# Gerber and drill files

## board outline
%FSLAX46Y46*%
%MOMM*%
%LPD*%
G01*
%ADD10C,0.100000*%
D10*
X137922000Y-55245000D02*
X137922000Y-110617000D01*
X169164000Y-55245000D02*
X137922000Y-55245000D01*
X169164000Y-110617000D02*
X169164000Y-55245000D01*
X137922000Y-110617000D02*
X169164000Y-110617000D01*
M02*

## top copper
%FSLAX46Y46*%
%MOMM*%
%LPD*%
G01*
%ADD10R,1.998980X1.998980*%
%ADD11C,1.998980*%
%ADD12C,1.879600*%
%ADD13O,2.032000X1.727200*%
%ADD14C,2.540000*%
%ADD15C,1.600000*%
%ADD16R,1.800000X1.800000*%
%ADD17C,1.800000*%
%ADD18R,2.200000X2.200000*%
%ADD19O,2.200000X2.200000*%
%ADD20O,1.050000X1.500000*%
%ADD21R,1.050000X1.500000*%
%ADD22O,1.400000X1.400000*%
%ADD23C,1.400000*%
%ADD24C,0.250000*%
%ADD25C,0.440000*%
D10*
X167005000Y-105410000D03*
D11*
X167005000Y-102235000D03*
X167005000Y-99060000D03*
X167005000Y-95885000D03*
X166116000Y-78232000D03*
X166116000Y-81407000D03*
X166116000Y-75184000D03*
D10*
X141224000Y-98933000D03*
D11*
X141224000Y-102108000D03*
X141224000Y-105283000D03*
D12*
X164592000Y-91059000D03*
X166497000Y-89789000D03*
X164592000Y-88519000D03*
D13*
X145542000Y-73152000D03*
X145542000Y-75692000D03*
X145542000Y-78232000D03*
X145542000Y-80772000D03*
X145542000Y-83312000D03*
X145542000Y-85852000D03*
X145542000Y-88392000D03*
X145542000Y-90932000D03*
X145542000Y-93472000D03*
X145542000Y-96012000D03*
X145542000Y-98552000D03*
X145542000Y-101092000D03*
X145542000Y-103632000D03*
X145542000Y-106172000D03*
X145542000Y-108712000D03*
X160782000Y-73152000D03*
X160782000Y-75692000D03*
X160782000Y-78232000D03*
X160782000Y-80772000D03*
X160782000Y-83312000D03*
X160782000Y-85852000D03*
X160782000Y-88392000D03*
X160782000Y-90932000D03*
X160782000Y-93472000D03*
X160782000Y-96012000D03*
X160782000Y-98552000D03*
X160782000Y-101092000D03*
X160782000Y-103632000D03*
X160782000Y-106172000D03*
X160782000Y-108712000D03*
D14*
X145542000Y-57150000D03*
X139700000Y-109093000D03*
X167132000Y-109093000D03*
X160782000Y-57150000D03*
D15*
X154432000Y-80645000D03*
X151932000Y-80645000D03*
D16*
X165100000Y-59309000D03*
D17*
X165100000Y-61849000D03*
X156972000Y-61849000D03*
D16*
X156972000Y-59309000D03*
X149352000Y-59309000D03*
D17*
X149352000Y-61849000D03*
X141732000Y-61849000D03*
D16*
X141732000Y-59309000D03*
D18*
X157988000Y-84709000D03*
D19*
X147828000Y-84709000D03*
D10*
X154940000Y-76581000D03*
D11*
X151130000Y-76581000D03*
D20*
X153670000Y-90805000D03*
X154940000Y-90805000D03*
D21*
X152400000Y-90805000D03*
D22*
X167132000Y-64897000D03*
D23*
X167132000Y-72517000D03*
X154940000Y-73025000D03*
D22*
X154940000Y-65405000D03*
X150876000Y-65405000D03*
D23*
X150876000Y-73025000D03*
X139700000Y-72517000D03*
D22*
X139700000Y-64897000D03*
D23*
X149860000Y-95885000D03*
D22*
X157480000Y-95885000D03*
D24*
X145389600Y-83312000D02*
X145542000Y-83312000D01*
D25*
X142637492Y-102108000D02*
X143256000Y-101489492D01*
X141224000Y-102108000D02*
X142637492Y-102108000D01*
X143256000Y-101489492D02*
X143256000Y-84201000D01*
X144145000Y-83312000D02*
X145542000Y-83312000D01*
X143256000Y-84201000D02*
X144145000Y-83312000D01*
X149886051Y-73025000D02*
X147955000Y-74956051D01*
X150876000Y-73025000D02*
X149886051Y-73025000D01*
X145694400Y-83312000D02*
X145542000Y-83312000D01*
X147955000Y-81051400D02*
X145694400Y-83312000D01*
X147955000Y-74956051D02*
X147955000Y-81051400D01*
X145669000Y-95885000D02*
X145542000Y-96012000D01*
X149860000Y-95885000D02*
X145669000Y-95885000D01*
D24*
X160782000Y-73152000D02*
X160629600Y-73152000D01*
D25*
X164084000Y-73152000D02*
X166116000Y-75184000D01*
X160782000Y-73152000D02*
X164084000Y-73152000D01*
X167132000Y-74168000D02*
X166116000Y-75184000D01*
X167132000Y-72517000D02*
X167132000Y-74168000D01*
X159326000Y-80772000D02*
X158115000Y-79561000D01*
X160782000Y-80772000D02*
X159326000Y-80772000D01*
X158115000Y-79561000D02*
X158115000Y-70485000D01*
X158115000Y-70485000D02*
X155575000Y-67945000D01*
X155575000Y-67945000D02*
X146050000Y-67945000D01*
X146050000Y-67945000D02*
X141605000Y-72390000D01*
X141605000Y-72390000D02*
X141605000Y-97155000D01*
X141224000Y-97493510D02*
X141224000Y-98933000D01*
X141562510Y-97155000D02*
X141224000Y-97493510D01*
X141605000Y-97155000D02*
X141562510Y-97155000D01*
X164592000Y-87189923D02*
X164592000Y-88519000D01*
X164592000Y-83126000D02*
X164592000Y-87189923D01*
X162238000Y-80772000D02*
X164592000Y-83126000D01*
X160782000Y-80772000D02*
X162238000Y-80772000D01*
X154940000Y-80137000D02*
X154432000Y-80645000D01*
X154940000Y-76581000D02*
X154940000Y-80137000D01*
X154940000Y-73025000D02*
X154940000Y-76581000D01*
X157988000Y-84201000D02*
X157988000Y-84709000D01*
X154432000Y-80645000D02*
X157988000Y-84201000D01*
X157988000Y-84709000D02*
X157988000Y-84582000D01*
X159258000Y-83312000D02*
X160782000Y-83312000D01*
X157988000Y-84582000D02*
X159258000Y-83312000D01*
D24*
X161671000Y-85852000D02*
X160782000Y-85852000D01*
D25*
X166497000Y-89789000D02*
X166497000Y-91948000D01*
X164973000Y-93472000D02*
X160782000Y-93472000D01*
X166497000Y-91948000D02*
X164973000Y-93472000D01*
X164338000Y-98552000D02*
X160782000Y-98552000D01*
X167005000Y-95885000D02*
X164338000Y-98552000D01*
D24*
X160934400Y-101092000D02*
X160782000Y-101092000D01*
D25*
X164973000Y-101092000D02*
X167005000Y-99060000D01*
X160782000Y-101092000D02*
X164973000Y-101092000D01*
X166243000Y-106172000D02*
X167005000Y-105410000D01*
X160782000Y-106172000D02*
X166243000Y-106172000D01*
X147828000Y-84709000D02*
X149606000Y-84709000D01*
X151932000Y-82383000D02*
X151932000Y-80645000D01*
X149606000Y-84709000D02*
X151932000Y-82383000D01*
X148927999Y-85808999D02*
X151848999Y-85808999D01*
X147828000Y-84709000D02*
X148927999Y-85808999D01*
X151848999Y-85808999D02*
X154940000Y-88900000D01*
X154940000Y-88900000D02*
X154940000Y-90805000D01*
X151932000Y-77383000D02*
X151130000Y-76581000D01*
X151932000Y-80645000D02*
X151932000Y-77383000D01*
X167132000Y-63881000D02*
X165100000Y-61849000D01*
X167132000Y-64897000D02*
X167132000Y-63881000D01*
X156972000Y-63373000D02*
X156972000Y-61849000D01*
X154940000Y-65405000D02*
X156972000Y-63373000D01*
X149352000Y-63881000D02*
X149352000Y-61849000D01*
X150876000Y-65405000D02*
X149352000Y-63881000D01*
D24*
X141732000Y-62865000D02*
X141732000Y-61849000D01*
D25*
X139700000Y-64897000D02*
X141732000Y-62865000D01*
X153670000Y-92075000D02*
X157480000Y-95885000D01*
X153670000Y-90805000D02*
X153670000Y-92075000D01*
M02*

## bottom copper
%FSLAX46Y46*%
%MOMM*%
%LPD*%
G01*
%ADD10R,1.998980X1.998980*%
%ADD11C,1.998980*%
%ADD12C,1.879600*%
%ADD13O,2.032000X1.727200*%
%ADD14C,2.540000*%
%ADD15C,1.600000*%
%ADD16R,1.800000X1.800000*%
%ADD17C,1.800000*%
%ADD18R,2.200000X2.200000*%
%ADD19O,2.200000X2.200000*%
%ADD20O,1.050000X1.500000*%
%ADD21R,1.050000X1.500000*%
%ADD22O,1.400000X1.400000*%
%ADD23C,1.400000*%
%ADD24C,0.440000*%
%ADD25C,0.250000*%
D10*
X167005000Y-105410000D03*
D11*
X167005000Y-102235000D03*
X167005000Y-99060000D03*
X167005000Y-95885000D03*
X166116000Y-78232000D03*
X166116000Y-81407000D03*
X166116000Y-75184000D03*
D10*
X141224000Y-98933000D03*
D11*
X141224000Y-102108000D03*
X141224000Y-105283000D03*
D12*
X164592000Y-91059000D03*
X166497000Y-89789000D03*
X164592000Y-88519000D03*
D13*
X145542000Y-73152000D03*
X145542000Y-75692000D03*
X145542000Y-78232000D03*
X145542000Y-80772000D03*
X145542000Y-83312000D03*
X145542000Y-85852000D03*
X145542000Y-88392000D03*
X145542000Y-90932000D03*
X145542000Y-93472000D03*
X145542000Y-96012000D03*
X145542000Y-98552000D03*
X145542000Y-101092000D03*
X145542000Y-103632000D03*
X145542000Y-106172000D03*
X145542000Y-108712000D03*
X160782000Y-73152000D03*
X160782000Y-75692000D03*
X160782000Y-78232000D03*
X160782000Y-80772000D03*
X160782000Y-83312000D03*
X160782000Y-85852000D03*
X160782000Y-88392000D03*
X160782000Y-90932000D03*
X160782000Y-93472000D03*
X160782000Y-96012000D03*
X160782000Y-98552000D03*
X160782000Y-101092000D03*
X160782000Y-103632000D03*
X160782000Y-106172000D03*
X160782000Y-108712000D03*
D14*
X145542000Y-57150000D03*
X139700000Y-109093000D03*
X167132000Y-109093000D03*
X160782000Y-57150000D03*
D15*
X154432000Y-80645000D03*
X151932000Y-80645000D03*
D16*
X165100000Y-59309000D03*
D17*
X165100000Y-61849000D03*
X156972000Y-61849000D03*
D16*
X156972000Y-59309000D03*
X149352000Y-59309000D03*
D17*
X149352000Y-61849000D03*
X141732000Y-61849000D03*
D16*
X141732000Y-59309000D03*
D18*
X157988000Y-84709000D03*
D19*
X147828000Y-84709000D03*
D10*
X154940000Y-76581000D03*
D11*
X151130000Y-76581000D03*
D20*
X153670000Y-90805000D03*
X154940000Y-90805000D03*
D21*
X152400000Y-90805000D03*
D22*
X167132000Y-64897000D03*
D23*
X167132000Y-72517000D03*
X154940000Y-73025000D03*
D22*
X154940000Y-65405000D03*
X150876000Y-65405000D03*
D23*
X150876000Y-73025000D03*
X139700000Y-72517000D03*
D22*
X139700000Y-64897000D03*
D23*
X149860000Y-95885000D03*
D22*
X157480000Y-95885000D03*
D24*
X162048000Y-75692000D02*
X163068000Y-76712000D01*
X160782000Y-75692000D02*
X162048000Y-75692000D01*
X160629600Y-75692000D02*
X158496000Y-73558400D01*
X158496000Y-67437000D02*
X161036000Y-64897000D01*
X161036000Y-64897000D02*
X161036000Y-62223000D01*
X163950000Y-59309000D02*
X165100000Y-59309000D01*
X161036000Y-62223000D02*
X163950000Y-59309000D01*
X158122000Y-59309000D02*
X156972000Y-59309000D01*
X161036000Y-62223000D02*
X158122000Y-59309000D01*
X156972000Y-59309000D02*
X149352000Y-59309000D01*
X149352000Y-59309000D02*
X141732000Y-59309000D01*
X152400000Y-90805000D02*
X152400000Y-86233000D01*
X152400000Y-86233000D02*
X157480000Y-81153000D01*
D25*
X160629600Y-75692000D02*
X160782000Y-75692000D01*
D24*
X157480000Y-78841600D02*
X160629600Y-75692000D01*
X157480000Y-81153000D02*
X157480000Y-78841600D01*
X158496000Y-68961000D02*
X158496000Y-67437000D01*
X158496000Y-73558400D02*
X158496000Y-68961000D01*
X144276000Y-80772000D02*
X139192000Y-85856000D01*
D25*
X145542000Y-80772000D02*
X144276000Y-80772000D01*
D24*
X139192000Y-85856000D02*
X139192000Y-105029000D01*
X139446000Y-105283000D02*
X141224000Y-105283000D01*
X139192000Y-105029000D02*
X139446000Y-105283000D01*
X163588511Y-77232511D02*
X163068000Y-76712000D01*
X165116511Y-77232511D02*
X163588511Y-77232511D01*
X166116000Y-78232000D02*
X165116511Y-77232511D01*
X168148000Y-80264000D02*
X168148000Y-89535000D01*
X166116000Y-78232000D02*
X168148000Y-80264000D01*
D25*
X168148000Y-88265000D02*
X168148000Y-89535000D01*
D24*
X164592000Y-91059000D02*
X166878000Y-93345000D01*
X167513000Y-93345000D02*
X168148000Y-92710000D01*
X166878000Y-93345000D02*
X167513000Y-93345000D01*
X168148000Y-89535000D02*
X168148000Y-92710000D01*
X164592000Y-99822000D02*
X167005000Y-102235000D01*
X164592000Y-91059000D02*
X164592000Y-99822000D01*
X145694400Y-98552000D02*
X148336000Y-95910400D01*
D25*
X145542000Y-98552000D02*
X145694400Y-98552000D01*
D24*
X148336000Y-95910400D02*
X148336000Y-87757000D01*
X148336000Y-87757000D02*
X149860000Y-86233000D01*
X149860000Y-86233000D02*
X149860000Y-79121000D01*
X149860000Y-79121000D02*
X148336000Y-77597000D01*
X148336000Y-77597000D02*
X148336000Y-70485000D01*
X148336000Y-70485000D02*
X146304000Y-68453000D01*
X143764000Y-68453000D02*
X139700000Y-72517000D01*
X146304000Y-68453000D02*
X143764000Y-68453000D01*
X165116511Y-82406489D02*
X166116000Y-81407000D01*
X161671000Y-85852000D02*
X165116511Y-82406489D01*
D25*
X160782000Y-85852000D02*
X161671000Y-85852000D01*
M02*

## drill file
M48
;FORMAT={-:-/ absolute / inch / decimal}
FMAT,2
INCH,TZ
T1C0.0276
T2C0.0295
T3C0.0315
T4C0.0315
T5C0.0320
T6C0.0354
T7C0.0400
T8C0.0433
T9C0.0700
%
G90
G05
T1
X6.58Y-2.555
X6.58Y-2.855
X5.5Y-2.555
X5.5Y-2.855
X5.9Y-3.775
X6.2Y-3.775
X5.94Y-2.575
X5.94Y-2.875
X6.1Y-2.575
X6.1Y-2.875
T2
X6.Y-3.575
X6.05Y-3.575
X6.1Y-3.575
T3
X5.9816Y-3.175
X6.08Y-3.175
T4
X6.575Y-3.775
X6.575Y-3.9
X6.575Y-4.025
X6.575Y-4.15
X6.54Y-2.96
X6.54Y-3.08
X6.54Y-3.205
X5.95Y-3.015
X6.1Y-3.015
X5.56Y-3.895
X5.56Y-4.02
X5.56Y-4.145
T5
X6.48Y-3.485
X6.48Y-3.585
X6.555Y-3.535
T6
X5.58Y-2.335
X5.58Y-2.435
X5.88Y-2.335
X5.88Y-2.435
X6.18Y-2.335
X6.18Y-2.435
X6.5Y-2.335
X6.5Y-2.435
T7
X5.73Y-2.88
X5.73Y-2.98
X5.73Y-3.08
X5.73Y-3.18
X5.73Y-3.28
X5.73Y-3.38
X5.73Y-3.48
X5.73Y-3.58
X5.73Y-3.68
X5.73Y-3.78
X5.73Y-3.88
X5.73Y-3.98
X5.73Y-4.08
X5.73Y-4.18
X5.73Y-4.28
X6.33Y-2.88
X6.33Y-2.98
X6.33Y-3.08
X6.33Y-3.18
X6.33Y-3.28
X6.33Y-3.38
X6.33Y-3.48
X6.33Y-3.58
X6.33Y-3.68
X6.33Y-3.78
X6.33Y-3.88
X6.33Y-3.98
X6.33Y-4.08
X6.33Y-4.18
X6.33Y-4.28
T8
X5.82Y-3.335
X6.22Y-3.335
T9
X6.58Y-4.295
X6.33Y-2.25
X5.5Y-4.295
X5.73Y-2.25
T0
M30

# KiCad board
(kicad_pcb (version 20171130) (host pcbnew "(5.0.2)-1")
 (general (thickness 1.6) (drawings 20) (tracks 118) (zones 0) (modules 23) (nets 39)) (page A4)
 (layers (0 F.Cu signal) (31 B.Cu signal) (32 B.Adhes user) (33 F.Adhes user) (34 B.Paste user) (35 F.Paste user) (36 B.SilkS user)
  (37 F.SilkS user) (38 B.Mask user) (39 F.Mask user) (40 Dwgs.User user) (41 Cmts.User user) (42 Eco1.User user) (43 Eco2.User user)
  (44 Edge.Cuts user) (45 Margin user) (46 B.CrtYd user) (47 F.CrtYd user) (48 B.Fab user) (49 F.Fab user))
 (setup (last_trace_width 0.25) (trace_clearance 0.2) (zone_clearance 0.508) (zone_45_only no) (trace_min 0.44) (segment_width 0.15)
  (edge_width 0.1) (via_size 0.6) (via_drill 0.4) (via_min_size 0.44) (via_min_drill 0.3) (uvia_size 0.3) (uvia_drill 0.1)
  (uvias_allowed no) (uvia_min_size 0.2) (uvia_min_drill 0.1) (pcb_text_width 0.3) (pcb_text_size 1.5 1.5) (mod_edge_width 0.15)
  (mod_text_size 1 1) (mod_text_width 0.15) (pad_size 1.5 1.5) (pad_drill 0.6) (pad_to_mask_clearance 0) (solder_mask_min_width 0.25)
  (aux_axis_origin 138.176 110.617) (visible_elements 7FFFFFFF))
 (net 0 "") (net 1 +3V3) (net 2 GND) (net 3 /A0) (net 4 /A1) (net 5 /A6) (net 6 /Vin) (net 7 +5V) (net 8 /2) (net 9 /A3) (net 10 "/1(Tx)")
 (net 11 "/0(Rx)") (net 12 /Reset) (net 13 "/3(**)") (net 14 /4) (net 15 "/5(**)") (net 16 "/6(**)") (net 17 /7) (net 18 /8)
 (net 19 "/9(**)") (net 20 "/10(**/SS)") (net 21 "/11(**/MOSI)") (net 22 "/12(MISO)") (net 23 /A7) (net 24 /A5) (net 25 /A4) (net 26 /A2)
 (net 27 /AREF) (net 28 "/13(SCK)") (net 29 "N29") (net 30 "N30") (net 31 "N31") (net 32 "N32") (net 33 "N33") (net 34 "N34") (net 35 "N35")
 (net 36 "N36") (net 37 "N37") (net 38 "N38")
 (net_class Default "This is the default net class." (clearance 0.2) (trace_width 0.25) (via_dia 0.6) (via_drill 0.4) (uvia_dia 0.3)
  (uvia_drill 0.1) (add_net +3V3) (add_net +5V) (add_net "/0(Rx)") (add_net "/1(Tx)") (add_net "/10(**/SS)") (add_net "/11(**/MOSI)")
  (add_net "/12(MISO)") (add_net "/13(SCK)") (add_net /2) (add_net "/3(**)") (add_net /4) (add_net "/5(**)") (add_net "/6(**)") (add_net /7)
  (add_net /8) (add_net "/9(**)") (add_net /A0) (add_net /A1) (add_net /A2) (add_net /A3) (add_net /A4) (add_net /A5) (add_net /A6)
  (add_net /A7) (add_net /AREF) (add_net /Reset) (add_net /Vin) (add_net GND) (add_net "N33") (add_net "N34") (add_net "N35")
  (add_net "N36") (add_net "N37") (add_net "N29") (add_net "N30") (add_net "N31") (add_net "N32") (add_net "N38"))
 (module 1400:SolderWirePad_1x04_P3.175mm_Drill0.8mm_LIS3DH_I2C (layer F.Cu) (at 167.005 105.41 90)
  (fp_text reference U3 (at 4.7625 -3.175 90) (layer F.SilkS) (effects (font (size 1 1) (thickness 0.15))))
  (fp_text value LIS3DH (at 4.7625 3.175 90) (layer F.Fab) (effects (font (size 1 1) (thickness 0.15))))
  (pad 14 thru_hole rect (at 0 0 90) (size 1.99898 1.99898) (drill 0.8001) (layers *.Cu *.Mask) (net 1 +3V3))
  (pad 5 thru_hole circle (at 3.175 0 90) (size 1.99898 1.99898) (drill 0.8001) (layers *.Cu *.Mask) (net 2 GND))
  (pad 6 thru_hole circle (at 6.35 0 180) (size 1.99898 1.99898) (drill 0.8001) (layers *.Cu *.Mask) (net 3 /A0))
  (pad 4 thru_hole circle (at 9.525 0 90) (size 1.99898 1.99898) (drill 0.8001) (layers *.Cu *.Mask) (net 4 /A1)))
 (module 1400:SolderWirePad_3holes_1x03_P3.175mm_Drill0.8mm (layer F.Cu) (at 166.116 75.057 270)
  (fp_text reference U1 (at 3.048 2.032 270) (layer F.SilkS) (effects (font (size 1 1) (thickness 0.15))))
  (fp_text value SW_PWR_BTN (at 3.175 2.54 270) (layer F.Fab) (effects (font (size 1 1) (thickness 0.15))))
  (pad 3 thru_hole circle (at 3.175 0 270) (size 1.99898 1.99898) (drill 0.8001) (layers *.Cu *.Mask) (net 2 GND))
  (pad 4 thru_hole circle (at 6.35 0 270) (size 1.99898 1.99898) (drill 0.8001) (layers *.Cu *.Mask) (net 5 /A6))
  (pad 2 thru_hole circle (at 0.127 0 270) (size 1.99898 1.99898) (drill 0.8001) (layers *.Cu *.Mask) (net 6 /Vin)))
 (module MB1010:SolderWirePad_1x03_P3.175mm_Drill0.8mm (layer F.Cu) (at 141.224 98.933 270)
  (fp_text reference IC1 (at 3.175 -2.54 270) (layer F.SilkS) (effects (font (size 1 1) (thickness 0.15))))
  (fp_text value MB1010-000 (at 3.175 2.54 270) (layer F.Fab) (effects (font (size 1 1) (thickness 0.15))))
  (pad 6 thru_hole rect (at 0 0 270) (size 1.99898 1.99898) (drill 0.8001) (layers *.Cu *.Mask) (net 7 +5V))
  (pad 2 thru_hole circle (at 3.175 0 270) (size 1.99898 1.99898) (drill 0.8001) (layers *.Cu *.Mask) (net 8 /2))
  (pad 7 thru_hole circle (at 6.35 0 270) (size 1.99898 1.99898) (drill 0.8001) (layers *.Cu *.Mask) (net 2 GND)))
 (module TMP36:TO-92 (layer F.Cu) (at 164.592 89.789 270)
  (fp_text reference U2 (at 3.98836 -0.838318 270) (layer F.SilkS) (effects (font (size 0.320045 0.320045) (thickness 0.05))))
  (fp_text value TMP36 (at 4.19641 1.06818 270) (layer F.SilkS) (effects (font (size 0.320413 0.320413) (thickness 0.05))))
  (pad 3 thru_hole circle (at 1.27 0 270) (size 1.8796 1.8796) (drill 0.8128) (layers *.Cu *.Mask) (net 2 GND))
  (pad 2 thru_hole circle (at 0 -1.905 270) (size 1.8796 1.8796) (drill 0.8128) (layers *.Cu *.Mask) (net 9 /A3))
  (pad 1 thru_hole circle (at -1.27 0 270) (size 1.8796 1.8796) (drill 0.8128) (layers *.Cu *.Mask) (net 7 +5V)))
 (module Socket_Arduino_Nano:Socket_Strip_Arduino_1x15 (layer F.Cu) (at 145.542 73.152 270)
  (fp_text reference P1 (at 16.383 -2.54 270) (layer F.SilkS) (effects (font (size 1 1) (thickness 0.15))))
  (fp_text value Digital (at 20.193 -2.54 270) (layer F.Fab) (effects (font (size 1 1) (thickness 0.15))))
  (pad 1 thru_hole oval (at 0 0 270) (size 1.7272 2.032) (drill 1.016) (layers *.Cu *.Mask F.SilkS) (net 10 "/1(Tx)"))
  (pad 2 thru_hole oval (at 2.54 0 270) (size 1.7272 2.032) (drill 1.016) (layers *.Cu *.Mask F.SilkS) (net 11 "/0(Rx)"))
  (pad 3 thru_hole oval (at 5.08 0 270) (size 1.7272 2.032) (drill 1.016) (layers *.Cu *.Mask F.SilkS) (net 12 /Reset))
  (pad 4 thru_hole oval (at 7.62 0 270) (size 1.7272 2.032) (drill 1.016) (layers *.Cu *.Mask F.SilkS) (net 2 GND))
  (pad 5 thru_hole oval (at 10.16 0 270) (size 1.7272 2.032) (drill 1.016) (layers *.Cu *.Mask F.SilkS) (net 8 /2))
  (pad 6 thru_hole oval (at 12.7 0 270) (size 1.7272 2.032) (drill 1.016) (layers *.Cu *.Mask F.SilkS) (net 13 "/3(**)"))
  (pad 7 thru_hole oval (at 15.24 0 270) (size 1.7272 2.032) (drill 1.016) (layers *.Cu *.Mask F.SilkS) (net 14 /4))
  (pad 8 thru_hole oval (at 17.78 0 270) (size 1.7272 2.032) (drill 1.016) (layers *.Cu *.Mask F.SilkS) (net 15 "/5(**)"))
  (pad 9 thru_hole oval (at 20.32 0 270) (size 1.7272 2.032) (drill 1.016) (layers *.Cu *.Mask F.SilkS) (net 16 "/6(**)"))
  (pad 10 thru_hole oval (at 22.86 0 270) (size 1.7272 2.032) (drill 1.016) (layers *.Cu *.Mask F.SilkS) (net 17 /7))
  (pad 11 thru_hole oval (at 25.4 0 270) (size 1.7272 2.032) (drill 1.016) (layers *.Cu *.Mask F.SilkS) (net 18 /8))
  (pad 12 thru_hole oval (at 27.94 0 270) (size 1.7272 2.032) (drill 1.016) (layers *.Cu *.Mask F.SilkS) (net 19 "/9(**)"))
  (pad 13 thru_hole oval (at 30.48 0 270) (size 1.7272 2.032) (drill 1.016) (layers *.Cu *.Mask F.SilkS) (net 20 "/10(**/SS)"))
  (pad 14 thru_hole oval (at 33.02 0 270) (size 1.7272 2.032) (drill 1.016) (layers *.Cu *.Mask F.SilkS) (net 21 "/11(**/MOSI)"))
  (pad 15 thru_hole oval (at 35.56 0 270) (size 1.7272 2.032) (drill 1.016) (layers *.Cu *.Mask F.SilkS) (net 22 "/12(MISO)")))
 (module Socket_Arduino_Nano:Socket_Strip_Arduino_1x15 (layer F.Cu) (at 160.782 73.152 270)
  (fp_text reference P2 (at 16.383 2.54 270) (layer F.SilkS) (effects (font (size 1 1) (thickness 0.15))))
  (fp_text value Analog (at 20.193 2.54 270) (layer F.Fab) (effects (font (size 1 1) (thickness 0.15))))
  (pad 1 thru_hole oval (at 0 0 270) (size 1.7272 2.032) (drill 1.016) (layers *.Cu *.Mask F.SilkS) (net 6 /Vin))
  (pad 2 thru_hole oval (at 2.54 0 270) (size 1.7272 2.032) (drill 1.016) (layers *.Cu *.Mask F.SilkS) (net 2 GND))
  (pad 3 thru_hole oval (at 5.08 0 270) (size 1.7272 2.032) (drill 1.016) (layers *.Cu *.Mask F.SilkS) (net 12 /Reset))
  (pad 4 thru_hole oval (at 7.62 0 270) (size 1.7272 2.032) (drill 1.016) (layers *.Cu *.Mask F.SilkS) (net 7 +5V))
  (pad 5 thru_hole oval (at 10.16 0 270) (size 1.7272 2.032) (drill 1.016) (layers *.Cu *.Mask F.SilkS) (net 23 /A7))
  (pad 6 thru_hole oval (at 12.7 0 270) (size 1.7272 2.032) (drill 1.016) (layers *.Cu *.Mask F.SilkS) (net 5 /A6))
  (pad 7 thru_hole oval (at 15.24 0 270) (size 1.7272 2.032) (drill 1.016) (layers *.Cu *.Mask F.SilkS) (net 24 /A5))
  (pad 8 thru_hole oval (at 17.78 0 270) (size 1.7272 2.032) (drill 1.016) (layers *.Cu *.Mask F.SilkS) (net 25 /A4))
  (pad 9 thru_hole oval (at 20.32 0 270) (size 1.7272 2.032) (drill 1.016) (layers *.Cu *.Mask F.SilkS) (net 9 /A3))
  (pad 10 thru_hole oval (at 22.86 0 270) (size 1.7272 2.032) (drill 1.016) (layers *.Cu *.Mask F.SilkS) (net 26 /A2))
  (pad 11 thru_hole oval (at 25.4 0 270) (size 1.7272 2.032) (drill 1.016) (layers *.Cu *.Mask F.SilkS) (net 4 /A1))
  (pad 12 thru_hole oval (at 27.94 0 270) (size 1.7272 2.032) (drill 1.016) (layers *.Cu *.Mask F.SilkS) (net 3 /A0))
  (pad 13 thru_hole oval (at 30.48 0 270) (size 1.7272 2.032) (drill 1.016) (layers *.Cu *.Mask F.SilkS) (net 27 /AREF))
  (pad 14 thru_hole oval (at 33.02 0 270) (size 1.7272 2.032) (drill 1.016) (layers *.Cu *.Mask F.SilkS) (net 1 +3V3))
  (pad 15 thru_hole oval (at 35.56 0 270) (size 1.7272 2.032) (drill 1.016) (layers *.Cu *.Mask F.SilkS) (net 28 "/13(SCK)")))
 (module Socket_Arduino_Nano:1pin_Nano (layer F.Cu) (at 145.542 57.15)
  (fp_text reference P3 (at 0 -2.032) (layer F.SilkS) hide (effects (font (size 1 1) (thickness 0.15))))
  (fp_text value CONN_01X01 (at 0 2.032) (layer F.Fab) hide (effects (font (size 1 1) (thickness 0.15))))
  (pad 1 thru_hole circle (at 0 0) (size 2.54 2.54) (drill 1.778) (layers *.Cu *.Mask F.SilkS) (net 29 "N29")))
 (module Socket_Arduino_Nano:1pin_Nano (layer F.Cu) (at 139.7 109.093)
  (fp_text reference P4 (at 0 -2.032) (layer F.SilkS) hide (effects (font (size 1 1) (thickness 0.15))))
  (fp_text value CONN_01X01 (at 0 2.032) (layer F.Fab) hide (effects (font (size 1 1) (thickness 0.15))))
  (pad 1 thru_hole circle (at 0 0) (size 2.54 2.54) (drill 1.778) (layers *.Cu *.Mask F.SilkS) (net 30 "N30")))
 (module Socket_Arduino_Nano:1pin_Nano (layer F.Cu) (at 167.132 109.093)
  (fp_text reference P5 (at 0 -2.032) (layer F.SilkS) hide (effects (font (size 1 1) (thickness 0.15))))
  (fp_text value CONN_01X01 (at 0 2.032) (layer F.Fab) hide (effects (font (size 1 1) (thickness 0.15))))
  (pad 1 thru_hole circle (at 0 0) (size 2.54 2.54) (drill 1.778) (layers *.Cu *.Mask F.SilkS) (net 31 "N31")))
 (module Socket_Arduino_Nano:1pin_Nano (layer F.Cu) (at 160.782 57.15)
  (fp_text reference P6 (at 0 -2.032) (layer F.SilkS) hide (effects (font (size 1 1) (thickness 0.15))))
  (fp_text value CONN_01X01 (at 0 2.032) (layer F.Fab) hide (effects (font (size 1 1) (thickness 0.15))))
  (pad 1 thru_hole circle (at 0 0) (size 2.54 2.54) (drill 1.778) (layers *.Cu *.Mask F.SilkS) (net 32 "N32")))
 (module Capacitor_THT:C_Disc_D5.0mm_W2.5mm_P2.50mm (layer F.Cu) (at 154.432 80.645 180)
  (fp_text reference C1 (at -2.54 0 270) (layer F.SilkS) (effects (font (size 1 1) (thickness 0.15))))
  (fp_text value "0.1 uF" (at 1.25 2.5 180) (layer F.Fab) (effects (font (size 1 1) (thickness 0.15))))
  (pad 1 thru_hole circle (at 0 0 180) (size 1.6 1.6) (drill 0.8) (layers *.Cu *.Mask) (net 23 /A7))
  (pad 2 thru_hole circle (at 2.5 0 180) (size 1.6 1.6) (drill 0.8) (layers *.Cu *.Mask) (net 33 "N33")))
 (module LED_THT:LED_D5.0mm (layer F.Cu) (at 165.1 59.309 270)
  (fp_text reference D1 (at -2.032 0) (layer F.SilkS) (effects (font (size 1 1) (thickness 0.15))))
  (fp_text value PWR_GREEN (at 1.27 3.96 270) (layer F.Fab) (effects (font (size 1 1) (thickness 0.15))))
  (pad 1 thru_hole rect (at 0 0 270) (size 1.8 1.8) (drill 0.9) (layers *.Cu *.Mask) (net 2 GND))
  (pad 2 thru_hole circle (at 2.54 0 270) (size 1.8 1.8) (drill 0.9) (layers *.Cu *.Mask) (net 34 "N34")))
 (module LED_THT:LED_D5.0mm (layer F.Cu) (at 156.972 59.309 270)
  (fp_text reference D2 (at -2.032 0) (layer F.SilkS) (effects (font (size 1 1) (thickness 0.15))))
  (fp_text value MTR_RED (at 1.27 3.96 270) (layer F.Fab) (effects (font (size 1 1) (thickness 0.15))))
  (pad 2 thru_hole circle (at 2.54 0 270) (size 1.8 1.8) (drill 0.9) (layers *.Cu *.Mask) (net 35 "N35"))
  (pad 1 thru_hole rect (at 0 0 270) (size 1.8 1.8) (drill 0.9) (layers *.Cu *.Mask) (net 2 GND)))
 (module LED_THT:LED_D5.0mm (layer F.Cu) (at 149.352 59.309 270)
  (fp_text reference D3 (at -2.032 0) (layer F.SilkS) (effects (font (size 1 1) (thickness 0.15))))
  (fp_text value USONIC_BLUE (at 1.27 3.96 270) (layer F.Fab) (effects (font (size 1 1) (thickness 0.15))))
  (pad 1 thru_hole rect (at 0 0 270) (size 1.8 1.8) (drill 0.9) (layers *.Cu *.Mask) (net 2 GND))
  (pad 2 thru_hole circle (at 2.54 0 270) (size 1.8 1.8) (drill 0.9) (layers *.Cu *.Mask) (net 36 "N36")))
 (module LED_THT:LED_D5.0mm (layer F.Cu) (at 141.732 59.309 270)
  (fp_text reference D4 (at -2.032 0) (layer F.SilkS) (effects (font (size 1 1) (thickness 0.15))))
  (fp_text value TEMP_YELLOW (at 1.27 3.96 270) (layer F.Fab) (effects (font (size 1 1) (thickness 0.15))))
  (pad 2 thru_hole circle (at 2.54 0 270) (size 1.8 1.8) (drill 0.9) (layers *.Cu *.Mask) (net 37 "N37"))
  (pad 1 thru_hole rect (at 0 0 270) (size 1.8 1.8) (drill 0.9) (layers *.Cu *.Mask) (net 2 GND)))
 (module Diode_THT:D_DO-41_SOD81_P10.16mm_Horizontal (layer F.Cu) (at 157.988 84.709 180)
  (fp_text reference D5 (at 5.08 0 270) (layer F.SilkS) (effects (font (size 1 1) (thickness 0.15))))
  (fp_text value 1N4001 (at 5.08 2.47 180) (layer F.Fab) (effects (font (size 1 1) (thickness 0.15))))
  (pad 1 thru_hole rect (at 0 0 180) (size 2.2 2.2) (drill 1.1) (layers *.Cu *.Mask) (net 23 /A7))
  (pad 2 thru_hole oval (at 10.16 0 180) (size 2.2 2.2) (drill 1.1) (layers *.Cu *.Mask) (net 33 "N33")))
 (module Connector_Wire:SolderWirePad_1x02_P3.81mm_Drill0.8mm (layer F.Cu) (at 154.94 76.581 180)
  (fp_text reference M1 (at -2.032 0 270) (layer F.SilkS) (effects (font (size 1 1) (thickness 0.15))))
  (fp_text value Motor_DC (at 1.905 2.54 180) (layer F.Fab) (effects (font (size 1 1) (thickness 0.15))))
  (pad 1 thru_hole rect (at 0 0 180) (size 1.99898 1.99898) (drill 0.8001) (layers *.Cu *.Mask) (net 23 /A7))
  (pad 2 thru_hole circle (at 3.81 0 180) (size 1.99898 1.99898) (drill 0.8001) (layers *.Cu *.Mask) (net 33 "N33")))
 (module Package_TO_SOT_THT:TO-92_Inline (layer F.Cu) (at 152.4 90.805)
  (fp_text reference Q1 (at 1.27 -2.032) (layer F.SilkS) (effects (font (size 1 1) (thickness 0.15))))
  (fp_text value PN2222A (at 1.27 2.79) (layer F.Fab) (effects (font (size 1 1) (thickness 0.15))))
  (pad 2 thru_hole oval (at 1.27 0) (size 1.05 1.5) (drill 0.75) (layers *.Cu *.Mask) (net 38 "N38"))
  (pad 3 thru_hole oval (at 2.54 0) (size 1.05 1.5) (drill 0.75) (layers *.Cu *.Mask) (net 33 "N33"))
  (pad 1 thru_hole rect (at 0 0) (size 1.05 1.5) (drill 0.75) (layers *.Cu *.Mask) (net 2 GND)))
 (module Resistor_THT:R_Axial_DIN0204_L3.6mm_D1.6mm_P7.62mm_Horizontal (layer F.Cu) (at 167.132 72.517 90)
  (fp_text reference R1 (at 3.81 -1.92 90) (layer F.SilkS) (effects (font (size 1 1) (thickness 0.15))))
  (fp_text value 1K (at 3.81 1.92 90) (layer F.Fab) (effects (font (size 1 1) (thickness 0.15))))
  (pad 2 thru_hole oval (at 7.62 0 90) (size 1.4 1.4) (drill 0.7) (layers *.Cu *.Mask) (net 34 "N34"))
  (pad 1 thru_hole circle (at 0 0 90) (size 1.4 1.4) (drill 0.7) (layers *.Cu *.Mask) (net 6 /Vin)))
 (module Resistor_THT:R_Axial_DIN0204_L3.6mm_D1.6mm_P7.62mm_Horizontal (layer F.Cu) (at 154.94 73.025 90)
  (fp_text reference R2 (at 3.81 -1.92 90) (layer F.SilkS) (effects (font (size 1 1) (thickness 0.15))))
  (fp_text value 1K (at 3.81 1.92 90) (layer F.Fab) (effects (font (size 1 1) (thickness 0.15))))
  (pad 1 thru_hole circle (at 0 0 90) (size 1.4 1.4) (drill 0.7) (layers *.Cu *.Mask) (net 23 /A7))
  (pad 2 thru_hole oval (at 7.62 0 90) (size 1.4 1.4) (drill 0.7) (layers *.Cu *.Mask) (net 35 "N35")))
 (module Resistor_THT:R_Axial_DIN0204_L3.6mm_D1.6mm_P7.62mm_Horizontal (layer F.Cu) (at 150.876 73.025 90)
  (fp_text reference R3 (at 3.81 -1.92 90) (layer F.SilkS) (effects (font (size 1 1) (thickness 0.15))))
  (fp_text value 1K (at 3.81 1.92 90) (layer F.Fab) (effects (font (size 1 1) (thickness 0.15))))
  (pad 2 thru_hole oval (at 7.62 0 90) (size 1.4 1.4) (drill 0.7) (layers *.Cu *.Mask) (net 36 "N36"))
  (pad 1 thru_hole circle (at 0 0 90) (size 1.4 1.4) (drill 0.7) (layers *.Cu *.Mask) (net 8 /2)))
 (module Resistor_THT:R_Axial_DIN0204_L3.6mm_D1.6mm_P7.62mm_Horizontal (layer F.Cu) (at 139.7 72.517 90)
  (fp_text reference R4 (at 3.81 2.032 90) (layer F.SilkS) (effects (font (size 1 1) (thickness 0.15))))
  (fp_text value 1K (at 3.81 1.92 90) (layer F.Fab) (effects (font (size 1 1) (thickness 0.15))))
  (pad 1 thru_hole circle (at 0 0 90) (size 1.4 1.4) (drill 0.7) (layers *.Cu *.Mask) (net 18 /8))
  (pad 2 thru_hole oval (at 7.62 0 90) (size 1.4 1.4) (drill 0.7) (layers *.Cu *.Mask) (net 37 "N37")))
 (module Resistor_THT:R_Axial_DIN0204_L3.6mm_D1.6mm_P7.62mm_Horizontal (layer F.Cu) (at 149.86 95.885)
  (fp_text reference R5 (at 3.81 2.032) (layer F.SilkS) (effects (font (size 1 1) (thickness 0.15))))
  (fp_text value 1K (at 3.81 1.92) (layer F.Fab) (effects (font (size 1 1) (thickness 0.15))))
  (pad 1 thru_hole circle (at 0 0) (size 1.4 1.4) (drill 0.7) (layers *.Cu *.Mask) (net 17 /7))
  (pad 2 thru_hole oval (at 7.62 0) (size 1.4 1.4) (drill 0.7) (layers *.Cu *.Mask) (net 38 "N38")))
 (gr_line (start 137.922 55.245) (end 137.922 110.617) (angle 90) (layer Edge.Cuts) (width 0.1))
 (gr_line (start 169.164 55.245) (end 137.922 55.245) (angle 90) (layer Edge.Cuts) (width 0.1))
 (gr_line (start 169.164 110.617) (end 169.164 55.245) (angle 90) (layer Edge.Cuts) (width 0.1))
 (gr_line (start 137.922 110.617) (end 169.164 110.617) (angle 90) (layer Edge.Cuts) (width 0.1))
 (segment (start 162.048 75.692) (end 163.068 76.712) (width 0.44) (layer B.Cu) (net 2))
 (segment (start 160.782 75.692) (end 162.048 75.692) (width 0.44) (layer B.Cu) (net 2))
 (segment (start 160.6296 75.692) (end 158.496 73.5584) (width 0.44) (layer B.Cu) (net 2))
 (segment (start 158.496 67.437) (end 161.036 64.897) (width 0.44) (layer B.Cu) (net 2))
 (segment (start 161.036 64.897) (end 161.036 62.223) (width 0.44) (layer B.Cu) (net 2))
 (segment (start 163.95 59.309) (end 165.1 59.309) (width 0.44) (layer B.Cu) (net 2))
 (segment (start 161.036 62.223) (end 163.95 59.309) (width 0.44) (layer B.Cu) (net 2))
 (segment (start 158.122 59.309) (end 156.972 59.309) (width 0.44) (layer B.Cu) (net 2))
 (segment (start 161.036 62.223) (end 158.122 59.309) (width 0.44) (layer B.Cu) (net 2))
 (segment (start 156.972 59.309) (end 149.352 59.309) (width 0.44) (layer B.Cu) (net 2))
 (segment (start 149.352 59.309) (end 141.732 59.309) (width 0.44) (layer B.Cu) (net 2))
 (segment (start 152.4 90.805) (end 152.4 86.233) (width 0.44) (layer B.Cu) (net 2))
 (segment (start 152.4 86.233) (end 157.48 81.153) (width 0.44) (layer B.Cu) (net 2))
 (segment (start 160.6296 75.692) (end 160.782 75.692) (width 0.25) (layer B.Cu) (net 2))
 (segment (start 157.48 78.8416) (end 160.6296 75.692) (width 0.44) (layer B.Cu) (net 2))
 (segment (start 157.48 81.153) (end 157.48 78.8416) (width 0.44) (layer B.Cu) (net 2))
 (segment (start 158.496 68.961) (end 158.496 67.437) (width 0.44) (layer B.Cu) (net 2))
 (segment (start 158.496 73.5584) (end 158.496 68.961) (width 0.44) (layer B.Cu) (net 2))
 (segment (start 144.276 80.772) (end 139.192 85.856) (width 0.44) (layer B.Cu) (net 2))
 (segment (start 145.542 80.772) (end 144.276 80.772) (width 0.25) (layer B.Cu) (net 2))
 (segment (start 139.192 85.856) (end 139.192 105.029) (width 0.44) (layer B.Cu) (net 2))
 (segment (start 139.446 105.283) (end 141.224 105.283) (width 0.44) (layer B.Cu) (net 2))
 (segment (start 139.192 105.029) (end 139.446 105.283) (width 0.44) (layer B.Cu) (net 2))
 (segment (start 163.588511 77.232511) (end 163.068 76.712) (width 0.44) (layer B.Cu) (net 2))
 (segment (start 165.116511 77.232511) (end 163.588511 77.232511) (width 0.44) (layer B.Cu) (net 2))
 (segment (start 166.116 78.232) (end 165.116511 77.232511) (width 0.44) (layer B.Cu) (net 2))
 (segment (start 168.148 80.264) (end 168.148 89.535) (width 0.44) (layer B.Cu) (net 2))
 (segment (start 166.116 78.232) (end 168.148 80.264) (width 0.44) (layer B.Cu) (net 2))
 (segment (start 168.148 88.265) (end 168.148 89.535) (width 0.25) (layer B.Cu) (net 2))
 (segment (start 164.592 91.059) (end 166.878 93.345) (width 0.44) (layer B.Cu) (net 2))
 (segment (start 167.513 93.345) (end 168.148 92.71) (width 0.44) (layer B.Cu) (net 2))
 (segment (start 166.878 93.345) (end 167.513 93.345) (width 0.44) (layer B.Cu) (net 2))
 (segment (start 168.148 89.535) (end 168.148 92.71) (width 0.44) (layer B.Cu) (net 2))
 (segment (start 164.592 99.822) (end 167.005 102.235) (width 0.44) (layer B.Cu) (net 2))
 (segment (start 164.592 91.059) (end 164.592 99.822) (width 0.44) (layer B.Cu) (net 2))
 (segment (start 145.3896 83.312) (end 145.542 83.312) (width 0.25) (layer F.Cu) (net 8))
 (segment (start 142.637492 102.108) (end 143.256 101.489492) (width 0.44) (layer F.Cu) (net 8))
 (segment (start 141.224 102.108) (end 142.637492 102.108) (width 0.44) (layer F.Cu) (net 8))
 (segment (start 143.256 101.489492) (end 143.256 84.201) (width 0.44) (layer F.Cu) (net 8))
 (segment (start 144.145 83.312) (end 145.542 83.312) (width 0.44) (layer F.Cu) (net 8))
 (segment (start 143.256 84.201) (end 144.145 83.312) (width 0.44) (layer F.Cu) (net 8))
 (segment (start 149.886051 73.025) (end 147.955 74.956051) (width 0.44) (layer F.Cu) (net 8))
 (segment (start 150.876 73.025) (end 149.886051 73.025) (width 0.44) (layer F.Cu) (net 8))
 (segment (start 145.6944 83.312) (end 145.542 83.312) (width 0.44) (layer F.Cu) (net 8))
 (segment (start 147.955 81.0514) (end 145.6944 83.312) (width 0.44) (layer F.Cu) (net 8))
 (segment (start 147.955 74.956051) (end 147.955 81.0514) (width 0.44) (layer F.Cu) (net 8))
 (segment (start 145.669 95.885) (end 145.542 96.012) (width 0.44) (layer F.Cu) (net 17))
 (segment (start 149.86 95.885) (end 145.669 95.885) (width 0.44) (layer F.Cu) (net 17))
 (segment (start 145.6944 98.552) (end 148.336 95.9104) (width 0.44) (layer B.Cu) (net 18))
 (segment (start 145.542 98.552) (end 145.6944 98.552) (width 0.25) (layer B.Cu) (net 18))
 (segment (start 148.336 95.9104) (end 148.336 87.757) (width 0.44) (layer B.Cu) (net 18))
 (segment (start 148.336 87.757) (end 149.86 86.233) (width 0.44) (layer B.Cu) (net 18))
 (segment (start 149.86 86.233) (end 149.86 79.121) (width 0.44) (layer B.Cu) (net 18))
 (segment (start 149.86 79.121) (end 148.336 77.597) (width 0.44) (layer B.Cu) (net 18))
 (segment (start 148.336 77.597) (end 148.336 70.485) (width 0.44) (layer B.Cu) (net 18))
 (segment (start 148.336 70.485) (end 146.304 68.453) (width 0.44) (layer B.Cu) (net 18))
 (segment (start 143.764 68.453) (end 139.7 72.517) (width 0.44) (layer B.Cu) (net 18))
 (segment (start 146.304 68.453) (end 143.764 68.453) (width 0.44) (layer B.Cu) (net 18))
 (segment (start 160.782 73.152) (end 160.6296 73.152) (width 0.25) (layer F.Cu) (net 6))
 (segment (start 164.084 73.152) (end 166.116 75.184) (width 0.44) (layer F.Cu) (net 6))
 (segment (start 160.782 73.152) (end 164.084 73.152) (width 0.44) (layer F.Cu) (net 6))
 (segment (start 167.132 74.168) (end 166.116 75.184) (width 0.44) (layer F.Cu) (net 6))
 (segment (start 167.132 72.517) (end 167.132 74.168) (width 0.44) (layer F.Cu) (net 6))
 (segment (start 159.326 80.772) (end 158.115 79.561) (width 0.44) (layer F.Cu) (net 7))
 (segment (start 160.782 80.772) (end 159.326 80.772) (width 0.44) (layer F.Cu) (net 7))
 (segment (start 158.115 79.561) (end 158.115 70.485) (width 0.44) (layer F.Cu) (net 7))
 (segment (start 158.115 70.485) (end 155.575 67.945) (width 0.44) (layer F.Cu) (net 7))
 (segment (start 155.575 67.945) (end 146.05 67.945) (width 0.44) (layer F.Cu) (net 7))
 (segment (start 146.05 67.945) (end 141.605 72.39) (width 0.44) (layer F.Cu) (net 7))
 (segment (start 141.605 72.39) (end 141.605 97.155) (width 0.44) (layer F.Cu) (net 7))
 (segment (start 141.224 97.49351) (end 141.224 98.933) (width 0.44) (layer F.Cu) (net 7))
 (segment (start 141.56251 97.155) (end 141.224 97.49351) (width 0.44) (layer F.Cu) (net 7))
 (segment (start 141.605 97.155) (end 141.56251 97.155) (width 0.44) (layer F.Cu) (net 7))
 (segment (start 164.592 87.189923) (end 164.592 88.519) (width 0.44) (layer F.Cu) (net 7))
 (segment (start 164.592 83.126) (end 164.592 87.189923) (width 0.44) (layer F.Cu) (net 7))
 (segment (start 162.238 80.772) (end 164.592 83.126) (width 0.44) (layer F.Cu) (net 7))
 (segment (start 160.782 80.772) (end 162.238 80.772) (width 0.44) (layer F.Cu) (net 7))
 (segment (start 154.94 80.137) (end 154.432 80.645) (width 0.44) (layer F.Cu) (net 23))
 (segment (start 154.94 76.581) (end 154.94 80.137) (width 0.44) (layer F.Cu) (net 23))
 (segment (start 154.94 73.025) (end 154.94 76.581) (width 0.44) (layer F.Cu) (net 23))
 (segment (start 157.988 84.201) (end 157.988 84.709) (width 0.44) (layer F.Cu) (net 23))
 (segment (start 154.432 80.645) (end 157.988 84.201) (width 0.44) (layer F.Cu) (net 23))
 (segment (start 157.988 84.709) (end 157.988 84.582) (width 0.44) (layer F.Cu) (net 23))
 (segment (start 159.258 83.312) (end 160.782 83.312) (width 0.44) (layer F.Cu) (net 23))
 (segment (start 157.988 84.582) (end 159.258 83.312) (width 0.44) (layer F.Cu) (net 23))
 (segment (start 161.671 85.852) (end 160.782 85.852) (width 0.25) (layer F.Cu) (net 5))
 (segment (start 165.116511 82.406489) (end 166.116 81.407) (width 0.44) (layer B.Cu) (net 5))
 (segment (start 161.671 85.852) (end 165.116511 82.406489) (width 0.44) (layer B.Cu) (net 5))
 (segment (start 160.782 85.852) (end 161.671 85.852) (width 0.25) (layer B.Cu) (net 5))
 (segment (start 166.497 89.789) (end 166.497 91.948) (width 0.44) (layer F.Cu) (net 9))
 (segment (start 164.973 93.472) (end 160.782 93.472) (width 0.44) (layer F.Cu) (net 9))
 (segment (start 166.497 91.948) (end 164.973 93.472) (width 0.44) (layer F.Cu) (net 9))
 (segment (start 164.338 98.552) (end 160.782 98.552) (width 0.44) (layer F.Cu) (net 4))
 (segment (start 167.005 95.885) (end 164.338 98.552) (width 0.44) (layer F.Cu) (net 4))
 (segment (start 160.9344 101.092) (end 160.782 101.092) (width 0.25) (layer F.Cu) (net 3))
 (segment (start 164.973 101.092) (end 167.005 99.06) (width 0.44) (layer F.Cu) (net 3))
 (segment (start 160.782 101.092) (end 164.973 101.092) (width 0.44) (layer F.Cu) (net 3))
 (segment (start 166.243 106.172) (end 167.005 105.41) (width 0.44) (layer F.Cu) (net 1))
 (segment (start 160.782 106.172) (end 166.243 106.172) (width 0.44) (layer F.Cu) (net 1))
 (segment (start 147.828 84.709) (end 149.606 84.709) (width 0.44) (layer F.Cu) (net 33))
 (segment (start 151.932 82.383) (end 151.932 80.645) (width 0.44) (layer F.Cu) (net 33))
 (segment (start 149.606 84.709) (end 151.932 82.383) (width 0.44) (layer F.Cu) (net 33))
 (segment (start 148.927999 85.808999) (end 151.848999 85.808999) (width 0.44) (layer F.Cu) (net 33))
 (segment (start 147.828 84.709) (end 148.927999 85.808999) (width 0.44) (layer F.Cu) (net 33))
 (segment (start 151.848999 85.808999) (end 154.94 88.9) (width 0.44) (layer F.Cu) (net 33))
 (segment (start 154.94 88.9) (end 154.94 90.805) (width 0.44) (layer F.Cu) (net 33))
 (segment (start 151.932 77.383) (end 151.13 76.581) (width 0.44) (layer F.Cu) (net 33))
 (segment (start 151.932 80.645) (end 151.932 77.383) (width 0.44) (layer F.Cu) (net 33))
 (segment (start 167.132 63.881) (end 165.1 61.849) (width 0.44) (layer F.Cu) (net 34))
 (segment (start 167.132 64.897) (end 167.132 63.881) (width 0.44) (layer F.Cu) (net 34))
 (segment (start 156.972 63.373) (end 156.972 61.849) (width 0.44) (layer F.Cu) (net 35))
 (segment (start 154.94 65.405) (end 156.972 63.373) (width 0.44) (layer F.Cu) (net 35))
 (segment (start 149.352 63.881) (end 149.352 61.849) (width 0.44) (layer F.Cu) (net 36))
 (segment (start 150.876 65.405) (end 149.352 63.881) (width 0.44) (layer F.Cu) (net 36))
 (segment (start 141.732 62.865) (end 141.732 61.849) (width 0.25) (layer F.Cu) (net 37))
 (segment (start 139.7 64.897) (end 141.732 62.865) (width 0.44) (layer F.Cu) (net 37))
 (segment (start 153.67 92.075) (end 157.48 95.885) (width 0.44) (layer F.Cu) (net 38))
 (segment (start 153.67 90.805) (end 153.67 92.075) (width 0.44) (layer F.Cu) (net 38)))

